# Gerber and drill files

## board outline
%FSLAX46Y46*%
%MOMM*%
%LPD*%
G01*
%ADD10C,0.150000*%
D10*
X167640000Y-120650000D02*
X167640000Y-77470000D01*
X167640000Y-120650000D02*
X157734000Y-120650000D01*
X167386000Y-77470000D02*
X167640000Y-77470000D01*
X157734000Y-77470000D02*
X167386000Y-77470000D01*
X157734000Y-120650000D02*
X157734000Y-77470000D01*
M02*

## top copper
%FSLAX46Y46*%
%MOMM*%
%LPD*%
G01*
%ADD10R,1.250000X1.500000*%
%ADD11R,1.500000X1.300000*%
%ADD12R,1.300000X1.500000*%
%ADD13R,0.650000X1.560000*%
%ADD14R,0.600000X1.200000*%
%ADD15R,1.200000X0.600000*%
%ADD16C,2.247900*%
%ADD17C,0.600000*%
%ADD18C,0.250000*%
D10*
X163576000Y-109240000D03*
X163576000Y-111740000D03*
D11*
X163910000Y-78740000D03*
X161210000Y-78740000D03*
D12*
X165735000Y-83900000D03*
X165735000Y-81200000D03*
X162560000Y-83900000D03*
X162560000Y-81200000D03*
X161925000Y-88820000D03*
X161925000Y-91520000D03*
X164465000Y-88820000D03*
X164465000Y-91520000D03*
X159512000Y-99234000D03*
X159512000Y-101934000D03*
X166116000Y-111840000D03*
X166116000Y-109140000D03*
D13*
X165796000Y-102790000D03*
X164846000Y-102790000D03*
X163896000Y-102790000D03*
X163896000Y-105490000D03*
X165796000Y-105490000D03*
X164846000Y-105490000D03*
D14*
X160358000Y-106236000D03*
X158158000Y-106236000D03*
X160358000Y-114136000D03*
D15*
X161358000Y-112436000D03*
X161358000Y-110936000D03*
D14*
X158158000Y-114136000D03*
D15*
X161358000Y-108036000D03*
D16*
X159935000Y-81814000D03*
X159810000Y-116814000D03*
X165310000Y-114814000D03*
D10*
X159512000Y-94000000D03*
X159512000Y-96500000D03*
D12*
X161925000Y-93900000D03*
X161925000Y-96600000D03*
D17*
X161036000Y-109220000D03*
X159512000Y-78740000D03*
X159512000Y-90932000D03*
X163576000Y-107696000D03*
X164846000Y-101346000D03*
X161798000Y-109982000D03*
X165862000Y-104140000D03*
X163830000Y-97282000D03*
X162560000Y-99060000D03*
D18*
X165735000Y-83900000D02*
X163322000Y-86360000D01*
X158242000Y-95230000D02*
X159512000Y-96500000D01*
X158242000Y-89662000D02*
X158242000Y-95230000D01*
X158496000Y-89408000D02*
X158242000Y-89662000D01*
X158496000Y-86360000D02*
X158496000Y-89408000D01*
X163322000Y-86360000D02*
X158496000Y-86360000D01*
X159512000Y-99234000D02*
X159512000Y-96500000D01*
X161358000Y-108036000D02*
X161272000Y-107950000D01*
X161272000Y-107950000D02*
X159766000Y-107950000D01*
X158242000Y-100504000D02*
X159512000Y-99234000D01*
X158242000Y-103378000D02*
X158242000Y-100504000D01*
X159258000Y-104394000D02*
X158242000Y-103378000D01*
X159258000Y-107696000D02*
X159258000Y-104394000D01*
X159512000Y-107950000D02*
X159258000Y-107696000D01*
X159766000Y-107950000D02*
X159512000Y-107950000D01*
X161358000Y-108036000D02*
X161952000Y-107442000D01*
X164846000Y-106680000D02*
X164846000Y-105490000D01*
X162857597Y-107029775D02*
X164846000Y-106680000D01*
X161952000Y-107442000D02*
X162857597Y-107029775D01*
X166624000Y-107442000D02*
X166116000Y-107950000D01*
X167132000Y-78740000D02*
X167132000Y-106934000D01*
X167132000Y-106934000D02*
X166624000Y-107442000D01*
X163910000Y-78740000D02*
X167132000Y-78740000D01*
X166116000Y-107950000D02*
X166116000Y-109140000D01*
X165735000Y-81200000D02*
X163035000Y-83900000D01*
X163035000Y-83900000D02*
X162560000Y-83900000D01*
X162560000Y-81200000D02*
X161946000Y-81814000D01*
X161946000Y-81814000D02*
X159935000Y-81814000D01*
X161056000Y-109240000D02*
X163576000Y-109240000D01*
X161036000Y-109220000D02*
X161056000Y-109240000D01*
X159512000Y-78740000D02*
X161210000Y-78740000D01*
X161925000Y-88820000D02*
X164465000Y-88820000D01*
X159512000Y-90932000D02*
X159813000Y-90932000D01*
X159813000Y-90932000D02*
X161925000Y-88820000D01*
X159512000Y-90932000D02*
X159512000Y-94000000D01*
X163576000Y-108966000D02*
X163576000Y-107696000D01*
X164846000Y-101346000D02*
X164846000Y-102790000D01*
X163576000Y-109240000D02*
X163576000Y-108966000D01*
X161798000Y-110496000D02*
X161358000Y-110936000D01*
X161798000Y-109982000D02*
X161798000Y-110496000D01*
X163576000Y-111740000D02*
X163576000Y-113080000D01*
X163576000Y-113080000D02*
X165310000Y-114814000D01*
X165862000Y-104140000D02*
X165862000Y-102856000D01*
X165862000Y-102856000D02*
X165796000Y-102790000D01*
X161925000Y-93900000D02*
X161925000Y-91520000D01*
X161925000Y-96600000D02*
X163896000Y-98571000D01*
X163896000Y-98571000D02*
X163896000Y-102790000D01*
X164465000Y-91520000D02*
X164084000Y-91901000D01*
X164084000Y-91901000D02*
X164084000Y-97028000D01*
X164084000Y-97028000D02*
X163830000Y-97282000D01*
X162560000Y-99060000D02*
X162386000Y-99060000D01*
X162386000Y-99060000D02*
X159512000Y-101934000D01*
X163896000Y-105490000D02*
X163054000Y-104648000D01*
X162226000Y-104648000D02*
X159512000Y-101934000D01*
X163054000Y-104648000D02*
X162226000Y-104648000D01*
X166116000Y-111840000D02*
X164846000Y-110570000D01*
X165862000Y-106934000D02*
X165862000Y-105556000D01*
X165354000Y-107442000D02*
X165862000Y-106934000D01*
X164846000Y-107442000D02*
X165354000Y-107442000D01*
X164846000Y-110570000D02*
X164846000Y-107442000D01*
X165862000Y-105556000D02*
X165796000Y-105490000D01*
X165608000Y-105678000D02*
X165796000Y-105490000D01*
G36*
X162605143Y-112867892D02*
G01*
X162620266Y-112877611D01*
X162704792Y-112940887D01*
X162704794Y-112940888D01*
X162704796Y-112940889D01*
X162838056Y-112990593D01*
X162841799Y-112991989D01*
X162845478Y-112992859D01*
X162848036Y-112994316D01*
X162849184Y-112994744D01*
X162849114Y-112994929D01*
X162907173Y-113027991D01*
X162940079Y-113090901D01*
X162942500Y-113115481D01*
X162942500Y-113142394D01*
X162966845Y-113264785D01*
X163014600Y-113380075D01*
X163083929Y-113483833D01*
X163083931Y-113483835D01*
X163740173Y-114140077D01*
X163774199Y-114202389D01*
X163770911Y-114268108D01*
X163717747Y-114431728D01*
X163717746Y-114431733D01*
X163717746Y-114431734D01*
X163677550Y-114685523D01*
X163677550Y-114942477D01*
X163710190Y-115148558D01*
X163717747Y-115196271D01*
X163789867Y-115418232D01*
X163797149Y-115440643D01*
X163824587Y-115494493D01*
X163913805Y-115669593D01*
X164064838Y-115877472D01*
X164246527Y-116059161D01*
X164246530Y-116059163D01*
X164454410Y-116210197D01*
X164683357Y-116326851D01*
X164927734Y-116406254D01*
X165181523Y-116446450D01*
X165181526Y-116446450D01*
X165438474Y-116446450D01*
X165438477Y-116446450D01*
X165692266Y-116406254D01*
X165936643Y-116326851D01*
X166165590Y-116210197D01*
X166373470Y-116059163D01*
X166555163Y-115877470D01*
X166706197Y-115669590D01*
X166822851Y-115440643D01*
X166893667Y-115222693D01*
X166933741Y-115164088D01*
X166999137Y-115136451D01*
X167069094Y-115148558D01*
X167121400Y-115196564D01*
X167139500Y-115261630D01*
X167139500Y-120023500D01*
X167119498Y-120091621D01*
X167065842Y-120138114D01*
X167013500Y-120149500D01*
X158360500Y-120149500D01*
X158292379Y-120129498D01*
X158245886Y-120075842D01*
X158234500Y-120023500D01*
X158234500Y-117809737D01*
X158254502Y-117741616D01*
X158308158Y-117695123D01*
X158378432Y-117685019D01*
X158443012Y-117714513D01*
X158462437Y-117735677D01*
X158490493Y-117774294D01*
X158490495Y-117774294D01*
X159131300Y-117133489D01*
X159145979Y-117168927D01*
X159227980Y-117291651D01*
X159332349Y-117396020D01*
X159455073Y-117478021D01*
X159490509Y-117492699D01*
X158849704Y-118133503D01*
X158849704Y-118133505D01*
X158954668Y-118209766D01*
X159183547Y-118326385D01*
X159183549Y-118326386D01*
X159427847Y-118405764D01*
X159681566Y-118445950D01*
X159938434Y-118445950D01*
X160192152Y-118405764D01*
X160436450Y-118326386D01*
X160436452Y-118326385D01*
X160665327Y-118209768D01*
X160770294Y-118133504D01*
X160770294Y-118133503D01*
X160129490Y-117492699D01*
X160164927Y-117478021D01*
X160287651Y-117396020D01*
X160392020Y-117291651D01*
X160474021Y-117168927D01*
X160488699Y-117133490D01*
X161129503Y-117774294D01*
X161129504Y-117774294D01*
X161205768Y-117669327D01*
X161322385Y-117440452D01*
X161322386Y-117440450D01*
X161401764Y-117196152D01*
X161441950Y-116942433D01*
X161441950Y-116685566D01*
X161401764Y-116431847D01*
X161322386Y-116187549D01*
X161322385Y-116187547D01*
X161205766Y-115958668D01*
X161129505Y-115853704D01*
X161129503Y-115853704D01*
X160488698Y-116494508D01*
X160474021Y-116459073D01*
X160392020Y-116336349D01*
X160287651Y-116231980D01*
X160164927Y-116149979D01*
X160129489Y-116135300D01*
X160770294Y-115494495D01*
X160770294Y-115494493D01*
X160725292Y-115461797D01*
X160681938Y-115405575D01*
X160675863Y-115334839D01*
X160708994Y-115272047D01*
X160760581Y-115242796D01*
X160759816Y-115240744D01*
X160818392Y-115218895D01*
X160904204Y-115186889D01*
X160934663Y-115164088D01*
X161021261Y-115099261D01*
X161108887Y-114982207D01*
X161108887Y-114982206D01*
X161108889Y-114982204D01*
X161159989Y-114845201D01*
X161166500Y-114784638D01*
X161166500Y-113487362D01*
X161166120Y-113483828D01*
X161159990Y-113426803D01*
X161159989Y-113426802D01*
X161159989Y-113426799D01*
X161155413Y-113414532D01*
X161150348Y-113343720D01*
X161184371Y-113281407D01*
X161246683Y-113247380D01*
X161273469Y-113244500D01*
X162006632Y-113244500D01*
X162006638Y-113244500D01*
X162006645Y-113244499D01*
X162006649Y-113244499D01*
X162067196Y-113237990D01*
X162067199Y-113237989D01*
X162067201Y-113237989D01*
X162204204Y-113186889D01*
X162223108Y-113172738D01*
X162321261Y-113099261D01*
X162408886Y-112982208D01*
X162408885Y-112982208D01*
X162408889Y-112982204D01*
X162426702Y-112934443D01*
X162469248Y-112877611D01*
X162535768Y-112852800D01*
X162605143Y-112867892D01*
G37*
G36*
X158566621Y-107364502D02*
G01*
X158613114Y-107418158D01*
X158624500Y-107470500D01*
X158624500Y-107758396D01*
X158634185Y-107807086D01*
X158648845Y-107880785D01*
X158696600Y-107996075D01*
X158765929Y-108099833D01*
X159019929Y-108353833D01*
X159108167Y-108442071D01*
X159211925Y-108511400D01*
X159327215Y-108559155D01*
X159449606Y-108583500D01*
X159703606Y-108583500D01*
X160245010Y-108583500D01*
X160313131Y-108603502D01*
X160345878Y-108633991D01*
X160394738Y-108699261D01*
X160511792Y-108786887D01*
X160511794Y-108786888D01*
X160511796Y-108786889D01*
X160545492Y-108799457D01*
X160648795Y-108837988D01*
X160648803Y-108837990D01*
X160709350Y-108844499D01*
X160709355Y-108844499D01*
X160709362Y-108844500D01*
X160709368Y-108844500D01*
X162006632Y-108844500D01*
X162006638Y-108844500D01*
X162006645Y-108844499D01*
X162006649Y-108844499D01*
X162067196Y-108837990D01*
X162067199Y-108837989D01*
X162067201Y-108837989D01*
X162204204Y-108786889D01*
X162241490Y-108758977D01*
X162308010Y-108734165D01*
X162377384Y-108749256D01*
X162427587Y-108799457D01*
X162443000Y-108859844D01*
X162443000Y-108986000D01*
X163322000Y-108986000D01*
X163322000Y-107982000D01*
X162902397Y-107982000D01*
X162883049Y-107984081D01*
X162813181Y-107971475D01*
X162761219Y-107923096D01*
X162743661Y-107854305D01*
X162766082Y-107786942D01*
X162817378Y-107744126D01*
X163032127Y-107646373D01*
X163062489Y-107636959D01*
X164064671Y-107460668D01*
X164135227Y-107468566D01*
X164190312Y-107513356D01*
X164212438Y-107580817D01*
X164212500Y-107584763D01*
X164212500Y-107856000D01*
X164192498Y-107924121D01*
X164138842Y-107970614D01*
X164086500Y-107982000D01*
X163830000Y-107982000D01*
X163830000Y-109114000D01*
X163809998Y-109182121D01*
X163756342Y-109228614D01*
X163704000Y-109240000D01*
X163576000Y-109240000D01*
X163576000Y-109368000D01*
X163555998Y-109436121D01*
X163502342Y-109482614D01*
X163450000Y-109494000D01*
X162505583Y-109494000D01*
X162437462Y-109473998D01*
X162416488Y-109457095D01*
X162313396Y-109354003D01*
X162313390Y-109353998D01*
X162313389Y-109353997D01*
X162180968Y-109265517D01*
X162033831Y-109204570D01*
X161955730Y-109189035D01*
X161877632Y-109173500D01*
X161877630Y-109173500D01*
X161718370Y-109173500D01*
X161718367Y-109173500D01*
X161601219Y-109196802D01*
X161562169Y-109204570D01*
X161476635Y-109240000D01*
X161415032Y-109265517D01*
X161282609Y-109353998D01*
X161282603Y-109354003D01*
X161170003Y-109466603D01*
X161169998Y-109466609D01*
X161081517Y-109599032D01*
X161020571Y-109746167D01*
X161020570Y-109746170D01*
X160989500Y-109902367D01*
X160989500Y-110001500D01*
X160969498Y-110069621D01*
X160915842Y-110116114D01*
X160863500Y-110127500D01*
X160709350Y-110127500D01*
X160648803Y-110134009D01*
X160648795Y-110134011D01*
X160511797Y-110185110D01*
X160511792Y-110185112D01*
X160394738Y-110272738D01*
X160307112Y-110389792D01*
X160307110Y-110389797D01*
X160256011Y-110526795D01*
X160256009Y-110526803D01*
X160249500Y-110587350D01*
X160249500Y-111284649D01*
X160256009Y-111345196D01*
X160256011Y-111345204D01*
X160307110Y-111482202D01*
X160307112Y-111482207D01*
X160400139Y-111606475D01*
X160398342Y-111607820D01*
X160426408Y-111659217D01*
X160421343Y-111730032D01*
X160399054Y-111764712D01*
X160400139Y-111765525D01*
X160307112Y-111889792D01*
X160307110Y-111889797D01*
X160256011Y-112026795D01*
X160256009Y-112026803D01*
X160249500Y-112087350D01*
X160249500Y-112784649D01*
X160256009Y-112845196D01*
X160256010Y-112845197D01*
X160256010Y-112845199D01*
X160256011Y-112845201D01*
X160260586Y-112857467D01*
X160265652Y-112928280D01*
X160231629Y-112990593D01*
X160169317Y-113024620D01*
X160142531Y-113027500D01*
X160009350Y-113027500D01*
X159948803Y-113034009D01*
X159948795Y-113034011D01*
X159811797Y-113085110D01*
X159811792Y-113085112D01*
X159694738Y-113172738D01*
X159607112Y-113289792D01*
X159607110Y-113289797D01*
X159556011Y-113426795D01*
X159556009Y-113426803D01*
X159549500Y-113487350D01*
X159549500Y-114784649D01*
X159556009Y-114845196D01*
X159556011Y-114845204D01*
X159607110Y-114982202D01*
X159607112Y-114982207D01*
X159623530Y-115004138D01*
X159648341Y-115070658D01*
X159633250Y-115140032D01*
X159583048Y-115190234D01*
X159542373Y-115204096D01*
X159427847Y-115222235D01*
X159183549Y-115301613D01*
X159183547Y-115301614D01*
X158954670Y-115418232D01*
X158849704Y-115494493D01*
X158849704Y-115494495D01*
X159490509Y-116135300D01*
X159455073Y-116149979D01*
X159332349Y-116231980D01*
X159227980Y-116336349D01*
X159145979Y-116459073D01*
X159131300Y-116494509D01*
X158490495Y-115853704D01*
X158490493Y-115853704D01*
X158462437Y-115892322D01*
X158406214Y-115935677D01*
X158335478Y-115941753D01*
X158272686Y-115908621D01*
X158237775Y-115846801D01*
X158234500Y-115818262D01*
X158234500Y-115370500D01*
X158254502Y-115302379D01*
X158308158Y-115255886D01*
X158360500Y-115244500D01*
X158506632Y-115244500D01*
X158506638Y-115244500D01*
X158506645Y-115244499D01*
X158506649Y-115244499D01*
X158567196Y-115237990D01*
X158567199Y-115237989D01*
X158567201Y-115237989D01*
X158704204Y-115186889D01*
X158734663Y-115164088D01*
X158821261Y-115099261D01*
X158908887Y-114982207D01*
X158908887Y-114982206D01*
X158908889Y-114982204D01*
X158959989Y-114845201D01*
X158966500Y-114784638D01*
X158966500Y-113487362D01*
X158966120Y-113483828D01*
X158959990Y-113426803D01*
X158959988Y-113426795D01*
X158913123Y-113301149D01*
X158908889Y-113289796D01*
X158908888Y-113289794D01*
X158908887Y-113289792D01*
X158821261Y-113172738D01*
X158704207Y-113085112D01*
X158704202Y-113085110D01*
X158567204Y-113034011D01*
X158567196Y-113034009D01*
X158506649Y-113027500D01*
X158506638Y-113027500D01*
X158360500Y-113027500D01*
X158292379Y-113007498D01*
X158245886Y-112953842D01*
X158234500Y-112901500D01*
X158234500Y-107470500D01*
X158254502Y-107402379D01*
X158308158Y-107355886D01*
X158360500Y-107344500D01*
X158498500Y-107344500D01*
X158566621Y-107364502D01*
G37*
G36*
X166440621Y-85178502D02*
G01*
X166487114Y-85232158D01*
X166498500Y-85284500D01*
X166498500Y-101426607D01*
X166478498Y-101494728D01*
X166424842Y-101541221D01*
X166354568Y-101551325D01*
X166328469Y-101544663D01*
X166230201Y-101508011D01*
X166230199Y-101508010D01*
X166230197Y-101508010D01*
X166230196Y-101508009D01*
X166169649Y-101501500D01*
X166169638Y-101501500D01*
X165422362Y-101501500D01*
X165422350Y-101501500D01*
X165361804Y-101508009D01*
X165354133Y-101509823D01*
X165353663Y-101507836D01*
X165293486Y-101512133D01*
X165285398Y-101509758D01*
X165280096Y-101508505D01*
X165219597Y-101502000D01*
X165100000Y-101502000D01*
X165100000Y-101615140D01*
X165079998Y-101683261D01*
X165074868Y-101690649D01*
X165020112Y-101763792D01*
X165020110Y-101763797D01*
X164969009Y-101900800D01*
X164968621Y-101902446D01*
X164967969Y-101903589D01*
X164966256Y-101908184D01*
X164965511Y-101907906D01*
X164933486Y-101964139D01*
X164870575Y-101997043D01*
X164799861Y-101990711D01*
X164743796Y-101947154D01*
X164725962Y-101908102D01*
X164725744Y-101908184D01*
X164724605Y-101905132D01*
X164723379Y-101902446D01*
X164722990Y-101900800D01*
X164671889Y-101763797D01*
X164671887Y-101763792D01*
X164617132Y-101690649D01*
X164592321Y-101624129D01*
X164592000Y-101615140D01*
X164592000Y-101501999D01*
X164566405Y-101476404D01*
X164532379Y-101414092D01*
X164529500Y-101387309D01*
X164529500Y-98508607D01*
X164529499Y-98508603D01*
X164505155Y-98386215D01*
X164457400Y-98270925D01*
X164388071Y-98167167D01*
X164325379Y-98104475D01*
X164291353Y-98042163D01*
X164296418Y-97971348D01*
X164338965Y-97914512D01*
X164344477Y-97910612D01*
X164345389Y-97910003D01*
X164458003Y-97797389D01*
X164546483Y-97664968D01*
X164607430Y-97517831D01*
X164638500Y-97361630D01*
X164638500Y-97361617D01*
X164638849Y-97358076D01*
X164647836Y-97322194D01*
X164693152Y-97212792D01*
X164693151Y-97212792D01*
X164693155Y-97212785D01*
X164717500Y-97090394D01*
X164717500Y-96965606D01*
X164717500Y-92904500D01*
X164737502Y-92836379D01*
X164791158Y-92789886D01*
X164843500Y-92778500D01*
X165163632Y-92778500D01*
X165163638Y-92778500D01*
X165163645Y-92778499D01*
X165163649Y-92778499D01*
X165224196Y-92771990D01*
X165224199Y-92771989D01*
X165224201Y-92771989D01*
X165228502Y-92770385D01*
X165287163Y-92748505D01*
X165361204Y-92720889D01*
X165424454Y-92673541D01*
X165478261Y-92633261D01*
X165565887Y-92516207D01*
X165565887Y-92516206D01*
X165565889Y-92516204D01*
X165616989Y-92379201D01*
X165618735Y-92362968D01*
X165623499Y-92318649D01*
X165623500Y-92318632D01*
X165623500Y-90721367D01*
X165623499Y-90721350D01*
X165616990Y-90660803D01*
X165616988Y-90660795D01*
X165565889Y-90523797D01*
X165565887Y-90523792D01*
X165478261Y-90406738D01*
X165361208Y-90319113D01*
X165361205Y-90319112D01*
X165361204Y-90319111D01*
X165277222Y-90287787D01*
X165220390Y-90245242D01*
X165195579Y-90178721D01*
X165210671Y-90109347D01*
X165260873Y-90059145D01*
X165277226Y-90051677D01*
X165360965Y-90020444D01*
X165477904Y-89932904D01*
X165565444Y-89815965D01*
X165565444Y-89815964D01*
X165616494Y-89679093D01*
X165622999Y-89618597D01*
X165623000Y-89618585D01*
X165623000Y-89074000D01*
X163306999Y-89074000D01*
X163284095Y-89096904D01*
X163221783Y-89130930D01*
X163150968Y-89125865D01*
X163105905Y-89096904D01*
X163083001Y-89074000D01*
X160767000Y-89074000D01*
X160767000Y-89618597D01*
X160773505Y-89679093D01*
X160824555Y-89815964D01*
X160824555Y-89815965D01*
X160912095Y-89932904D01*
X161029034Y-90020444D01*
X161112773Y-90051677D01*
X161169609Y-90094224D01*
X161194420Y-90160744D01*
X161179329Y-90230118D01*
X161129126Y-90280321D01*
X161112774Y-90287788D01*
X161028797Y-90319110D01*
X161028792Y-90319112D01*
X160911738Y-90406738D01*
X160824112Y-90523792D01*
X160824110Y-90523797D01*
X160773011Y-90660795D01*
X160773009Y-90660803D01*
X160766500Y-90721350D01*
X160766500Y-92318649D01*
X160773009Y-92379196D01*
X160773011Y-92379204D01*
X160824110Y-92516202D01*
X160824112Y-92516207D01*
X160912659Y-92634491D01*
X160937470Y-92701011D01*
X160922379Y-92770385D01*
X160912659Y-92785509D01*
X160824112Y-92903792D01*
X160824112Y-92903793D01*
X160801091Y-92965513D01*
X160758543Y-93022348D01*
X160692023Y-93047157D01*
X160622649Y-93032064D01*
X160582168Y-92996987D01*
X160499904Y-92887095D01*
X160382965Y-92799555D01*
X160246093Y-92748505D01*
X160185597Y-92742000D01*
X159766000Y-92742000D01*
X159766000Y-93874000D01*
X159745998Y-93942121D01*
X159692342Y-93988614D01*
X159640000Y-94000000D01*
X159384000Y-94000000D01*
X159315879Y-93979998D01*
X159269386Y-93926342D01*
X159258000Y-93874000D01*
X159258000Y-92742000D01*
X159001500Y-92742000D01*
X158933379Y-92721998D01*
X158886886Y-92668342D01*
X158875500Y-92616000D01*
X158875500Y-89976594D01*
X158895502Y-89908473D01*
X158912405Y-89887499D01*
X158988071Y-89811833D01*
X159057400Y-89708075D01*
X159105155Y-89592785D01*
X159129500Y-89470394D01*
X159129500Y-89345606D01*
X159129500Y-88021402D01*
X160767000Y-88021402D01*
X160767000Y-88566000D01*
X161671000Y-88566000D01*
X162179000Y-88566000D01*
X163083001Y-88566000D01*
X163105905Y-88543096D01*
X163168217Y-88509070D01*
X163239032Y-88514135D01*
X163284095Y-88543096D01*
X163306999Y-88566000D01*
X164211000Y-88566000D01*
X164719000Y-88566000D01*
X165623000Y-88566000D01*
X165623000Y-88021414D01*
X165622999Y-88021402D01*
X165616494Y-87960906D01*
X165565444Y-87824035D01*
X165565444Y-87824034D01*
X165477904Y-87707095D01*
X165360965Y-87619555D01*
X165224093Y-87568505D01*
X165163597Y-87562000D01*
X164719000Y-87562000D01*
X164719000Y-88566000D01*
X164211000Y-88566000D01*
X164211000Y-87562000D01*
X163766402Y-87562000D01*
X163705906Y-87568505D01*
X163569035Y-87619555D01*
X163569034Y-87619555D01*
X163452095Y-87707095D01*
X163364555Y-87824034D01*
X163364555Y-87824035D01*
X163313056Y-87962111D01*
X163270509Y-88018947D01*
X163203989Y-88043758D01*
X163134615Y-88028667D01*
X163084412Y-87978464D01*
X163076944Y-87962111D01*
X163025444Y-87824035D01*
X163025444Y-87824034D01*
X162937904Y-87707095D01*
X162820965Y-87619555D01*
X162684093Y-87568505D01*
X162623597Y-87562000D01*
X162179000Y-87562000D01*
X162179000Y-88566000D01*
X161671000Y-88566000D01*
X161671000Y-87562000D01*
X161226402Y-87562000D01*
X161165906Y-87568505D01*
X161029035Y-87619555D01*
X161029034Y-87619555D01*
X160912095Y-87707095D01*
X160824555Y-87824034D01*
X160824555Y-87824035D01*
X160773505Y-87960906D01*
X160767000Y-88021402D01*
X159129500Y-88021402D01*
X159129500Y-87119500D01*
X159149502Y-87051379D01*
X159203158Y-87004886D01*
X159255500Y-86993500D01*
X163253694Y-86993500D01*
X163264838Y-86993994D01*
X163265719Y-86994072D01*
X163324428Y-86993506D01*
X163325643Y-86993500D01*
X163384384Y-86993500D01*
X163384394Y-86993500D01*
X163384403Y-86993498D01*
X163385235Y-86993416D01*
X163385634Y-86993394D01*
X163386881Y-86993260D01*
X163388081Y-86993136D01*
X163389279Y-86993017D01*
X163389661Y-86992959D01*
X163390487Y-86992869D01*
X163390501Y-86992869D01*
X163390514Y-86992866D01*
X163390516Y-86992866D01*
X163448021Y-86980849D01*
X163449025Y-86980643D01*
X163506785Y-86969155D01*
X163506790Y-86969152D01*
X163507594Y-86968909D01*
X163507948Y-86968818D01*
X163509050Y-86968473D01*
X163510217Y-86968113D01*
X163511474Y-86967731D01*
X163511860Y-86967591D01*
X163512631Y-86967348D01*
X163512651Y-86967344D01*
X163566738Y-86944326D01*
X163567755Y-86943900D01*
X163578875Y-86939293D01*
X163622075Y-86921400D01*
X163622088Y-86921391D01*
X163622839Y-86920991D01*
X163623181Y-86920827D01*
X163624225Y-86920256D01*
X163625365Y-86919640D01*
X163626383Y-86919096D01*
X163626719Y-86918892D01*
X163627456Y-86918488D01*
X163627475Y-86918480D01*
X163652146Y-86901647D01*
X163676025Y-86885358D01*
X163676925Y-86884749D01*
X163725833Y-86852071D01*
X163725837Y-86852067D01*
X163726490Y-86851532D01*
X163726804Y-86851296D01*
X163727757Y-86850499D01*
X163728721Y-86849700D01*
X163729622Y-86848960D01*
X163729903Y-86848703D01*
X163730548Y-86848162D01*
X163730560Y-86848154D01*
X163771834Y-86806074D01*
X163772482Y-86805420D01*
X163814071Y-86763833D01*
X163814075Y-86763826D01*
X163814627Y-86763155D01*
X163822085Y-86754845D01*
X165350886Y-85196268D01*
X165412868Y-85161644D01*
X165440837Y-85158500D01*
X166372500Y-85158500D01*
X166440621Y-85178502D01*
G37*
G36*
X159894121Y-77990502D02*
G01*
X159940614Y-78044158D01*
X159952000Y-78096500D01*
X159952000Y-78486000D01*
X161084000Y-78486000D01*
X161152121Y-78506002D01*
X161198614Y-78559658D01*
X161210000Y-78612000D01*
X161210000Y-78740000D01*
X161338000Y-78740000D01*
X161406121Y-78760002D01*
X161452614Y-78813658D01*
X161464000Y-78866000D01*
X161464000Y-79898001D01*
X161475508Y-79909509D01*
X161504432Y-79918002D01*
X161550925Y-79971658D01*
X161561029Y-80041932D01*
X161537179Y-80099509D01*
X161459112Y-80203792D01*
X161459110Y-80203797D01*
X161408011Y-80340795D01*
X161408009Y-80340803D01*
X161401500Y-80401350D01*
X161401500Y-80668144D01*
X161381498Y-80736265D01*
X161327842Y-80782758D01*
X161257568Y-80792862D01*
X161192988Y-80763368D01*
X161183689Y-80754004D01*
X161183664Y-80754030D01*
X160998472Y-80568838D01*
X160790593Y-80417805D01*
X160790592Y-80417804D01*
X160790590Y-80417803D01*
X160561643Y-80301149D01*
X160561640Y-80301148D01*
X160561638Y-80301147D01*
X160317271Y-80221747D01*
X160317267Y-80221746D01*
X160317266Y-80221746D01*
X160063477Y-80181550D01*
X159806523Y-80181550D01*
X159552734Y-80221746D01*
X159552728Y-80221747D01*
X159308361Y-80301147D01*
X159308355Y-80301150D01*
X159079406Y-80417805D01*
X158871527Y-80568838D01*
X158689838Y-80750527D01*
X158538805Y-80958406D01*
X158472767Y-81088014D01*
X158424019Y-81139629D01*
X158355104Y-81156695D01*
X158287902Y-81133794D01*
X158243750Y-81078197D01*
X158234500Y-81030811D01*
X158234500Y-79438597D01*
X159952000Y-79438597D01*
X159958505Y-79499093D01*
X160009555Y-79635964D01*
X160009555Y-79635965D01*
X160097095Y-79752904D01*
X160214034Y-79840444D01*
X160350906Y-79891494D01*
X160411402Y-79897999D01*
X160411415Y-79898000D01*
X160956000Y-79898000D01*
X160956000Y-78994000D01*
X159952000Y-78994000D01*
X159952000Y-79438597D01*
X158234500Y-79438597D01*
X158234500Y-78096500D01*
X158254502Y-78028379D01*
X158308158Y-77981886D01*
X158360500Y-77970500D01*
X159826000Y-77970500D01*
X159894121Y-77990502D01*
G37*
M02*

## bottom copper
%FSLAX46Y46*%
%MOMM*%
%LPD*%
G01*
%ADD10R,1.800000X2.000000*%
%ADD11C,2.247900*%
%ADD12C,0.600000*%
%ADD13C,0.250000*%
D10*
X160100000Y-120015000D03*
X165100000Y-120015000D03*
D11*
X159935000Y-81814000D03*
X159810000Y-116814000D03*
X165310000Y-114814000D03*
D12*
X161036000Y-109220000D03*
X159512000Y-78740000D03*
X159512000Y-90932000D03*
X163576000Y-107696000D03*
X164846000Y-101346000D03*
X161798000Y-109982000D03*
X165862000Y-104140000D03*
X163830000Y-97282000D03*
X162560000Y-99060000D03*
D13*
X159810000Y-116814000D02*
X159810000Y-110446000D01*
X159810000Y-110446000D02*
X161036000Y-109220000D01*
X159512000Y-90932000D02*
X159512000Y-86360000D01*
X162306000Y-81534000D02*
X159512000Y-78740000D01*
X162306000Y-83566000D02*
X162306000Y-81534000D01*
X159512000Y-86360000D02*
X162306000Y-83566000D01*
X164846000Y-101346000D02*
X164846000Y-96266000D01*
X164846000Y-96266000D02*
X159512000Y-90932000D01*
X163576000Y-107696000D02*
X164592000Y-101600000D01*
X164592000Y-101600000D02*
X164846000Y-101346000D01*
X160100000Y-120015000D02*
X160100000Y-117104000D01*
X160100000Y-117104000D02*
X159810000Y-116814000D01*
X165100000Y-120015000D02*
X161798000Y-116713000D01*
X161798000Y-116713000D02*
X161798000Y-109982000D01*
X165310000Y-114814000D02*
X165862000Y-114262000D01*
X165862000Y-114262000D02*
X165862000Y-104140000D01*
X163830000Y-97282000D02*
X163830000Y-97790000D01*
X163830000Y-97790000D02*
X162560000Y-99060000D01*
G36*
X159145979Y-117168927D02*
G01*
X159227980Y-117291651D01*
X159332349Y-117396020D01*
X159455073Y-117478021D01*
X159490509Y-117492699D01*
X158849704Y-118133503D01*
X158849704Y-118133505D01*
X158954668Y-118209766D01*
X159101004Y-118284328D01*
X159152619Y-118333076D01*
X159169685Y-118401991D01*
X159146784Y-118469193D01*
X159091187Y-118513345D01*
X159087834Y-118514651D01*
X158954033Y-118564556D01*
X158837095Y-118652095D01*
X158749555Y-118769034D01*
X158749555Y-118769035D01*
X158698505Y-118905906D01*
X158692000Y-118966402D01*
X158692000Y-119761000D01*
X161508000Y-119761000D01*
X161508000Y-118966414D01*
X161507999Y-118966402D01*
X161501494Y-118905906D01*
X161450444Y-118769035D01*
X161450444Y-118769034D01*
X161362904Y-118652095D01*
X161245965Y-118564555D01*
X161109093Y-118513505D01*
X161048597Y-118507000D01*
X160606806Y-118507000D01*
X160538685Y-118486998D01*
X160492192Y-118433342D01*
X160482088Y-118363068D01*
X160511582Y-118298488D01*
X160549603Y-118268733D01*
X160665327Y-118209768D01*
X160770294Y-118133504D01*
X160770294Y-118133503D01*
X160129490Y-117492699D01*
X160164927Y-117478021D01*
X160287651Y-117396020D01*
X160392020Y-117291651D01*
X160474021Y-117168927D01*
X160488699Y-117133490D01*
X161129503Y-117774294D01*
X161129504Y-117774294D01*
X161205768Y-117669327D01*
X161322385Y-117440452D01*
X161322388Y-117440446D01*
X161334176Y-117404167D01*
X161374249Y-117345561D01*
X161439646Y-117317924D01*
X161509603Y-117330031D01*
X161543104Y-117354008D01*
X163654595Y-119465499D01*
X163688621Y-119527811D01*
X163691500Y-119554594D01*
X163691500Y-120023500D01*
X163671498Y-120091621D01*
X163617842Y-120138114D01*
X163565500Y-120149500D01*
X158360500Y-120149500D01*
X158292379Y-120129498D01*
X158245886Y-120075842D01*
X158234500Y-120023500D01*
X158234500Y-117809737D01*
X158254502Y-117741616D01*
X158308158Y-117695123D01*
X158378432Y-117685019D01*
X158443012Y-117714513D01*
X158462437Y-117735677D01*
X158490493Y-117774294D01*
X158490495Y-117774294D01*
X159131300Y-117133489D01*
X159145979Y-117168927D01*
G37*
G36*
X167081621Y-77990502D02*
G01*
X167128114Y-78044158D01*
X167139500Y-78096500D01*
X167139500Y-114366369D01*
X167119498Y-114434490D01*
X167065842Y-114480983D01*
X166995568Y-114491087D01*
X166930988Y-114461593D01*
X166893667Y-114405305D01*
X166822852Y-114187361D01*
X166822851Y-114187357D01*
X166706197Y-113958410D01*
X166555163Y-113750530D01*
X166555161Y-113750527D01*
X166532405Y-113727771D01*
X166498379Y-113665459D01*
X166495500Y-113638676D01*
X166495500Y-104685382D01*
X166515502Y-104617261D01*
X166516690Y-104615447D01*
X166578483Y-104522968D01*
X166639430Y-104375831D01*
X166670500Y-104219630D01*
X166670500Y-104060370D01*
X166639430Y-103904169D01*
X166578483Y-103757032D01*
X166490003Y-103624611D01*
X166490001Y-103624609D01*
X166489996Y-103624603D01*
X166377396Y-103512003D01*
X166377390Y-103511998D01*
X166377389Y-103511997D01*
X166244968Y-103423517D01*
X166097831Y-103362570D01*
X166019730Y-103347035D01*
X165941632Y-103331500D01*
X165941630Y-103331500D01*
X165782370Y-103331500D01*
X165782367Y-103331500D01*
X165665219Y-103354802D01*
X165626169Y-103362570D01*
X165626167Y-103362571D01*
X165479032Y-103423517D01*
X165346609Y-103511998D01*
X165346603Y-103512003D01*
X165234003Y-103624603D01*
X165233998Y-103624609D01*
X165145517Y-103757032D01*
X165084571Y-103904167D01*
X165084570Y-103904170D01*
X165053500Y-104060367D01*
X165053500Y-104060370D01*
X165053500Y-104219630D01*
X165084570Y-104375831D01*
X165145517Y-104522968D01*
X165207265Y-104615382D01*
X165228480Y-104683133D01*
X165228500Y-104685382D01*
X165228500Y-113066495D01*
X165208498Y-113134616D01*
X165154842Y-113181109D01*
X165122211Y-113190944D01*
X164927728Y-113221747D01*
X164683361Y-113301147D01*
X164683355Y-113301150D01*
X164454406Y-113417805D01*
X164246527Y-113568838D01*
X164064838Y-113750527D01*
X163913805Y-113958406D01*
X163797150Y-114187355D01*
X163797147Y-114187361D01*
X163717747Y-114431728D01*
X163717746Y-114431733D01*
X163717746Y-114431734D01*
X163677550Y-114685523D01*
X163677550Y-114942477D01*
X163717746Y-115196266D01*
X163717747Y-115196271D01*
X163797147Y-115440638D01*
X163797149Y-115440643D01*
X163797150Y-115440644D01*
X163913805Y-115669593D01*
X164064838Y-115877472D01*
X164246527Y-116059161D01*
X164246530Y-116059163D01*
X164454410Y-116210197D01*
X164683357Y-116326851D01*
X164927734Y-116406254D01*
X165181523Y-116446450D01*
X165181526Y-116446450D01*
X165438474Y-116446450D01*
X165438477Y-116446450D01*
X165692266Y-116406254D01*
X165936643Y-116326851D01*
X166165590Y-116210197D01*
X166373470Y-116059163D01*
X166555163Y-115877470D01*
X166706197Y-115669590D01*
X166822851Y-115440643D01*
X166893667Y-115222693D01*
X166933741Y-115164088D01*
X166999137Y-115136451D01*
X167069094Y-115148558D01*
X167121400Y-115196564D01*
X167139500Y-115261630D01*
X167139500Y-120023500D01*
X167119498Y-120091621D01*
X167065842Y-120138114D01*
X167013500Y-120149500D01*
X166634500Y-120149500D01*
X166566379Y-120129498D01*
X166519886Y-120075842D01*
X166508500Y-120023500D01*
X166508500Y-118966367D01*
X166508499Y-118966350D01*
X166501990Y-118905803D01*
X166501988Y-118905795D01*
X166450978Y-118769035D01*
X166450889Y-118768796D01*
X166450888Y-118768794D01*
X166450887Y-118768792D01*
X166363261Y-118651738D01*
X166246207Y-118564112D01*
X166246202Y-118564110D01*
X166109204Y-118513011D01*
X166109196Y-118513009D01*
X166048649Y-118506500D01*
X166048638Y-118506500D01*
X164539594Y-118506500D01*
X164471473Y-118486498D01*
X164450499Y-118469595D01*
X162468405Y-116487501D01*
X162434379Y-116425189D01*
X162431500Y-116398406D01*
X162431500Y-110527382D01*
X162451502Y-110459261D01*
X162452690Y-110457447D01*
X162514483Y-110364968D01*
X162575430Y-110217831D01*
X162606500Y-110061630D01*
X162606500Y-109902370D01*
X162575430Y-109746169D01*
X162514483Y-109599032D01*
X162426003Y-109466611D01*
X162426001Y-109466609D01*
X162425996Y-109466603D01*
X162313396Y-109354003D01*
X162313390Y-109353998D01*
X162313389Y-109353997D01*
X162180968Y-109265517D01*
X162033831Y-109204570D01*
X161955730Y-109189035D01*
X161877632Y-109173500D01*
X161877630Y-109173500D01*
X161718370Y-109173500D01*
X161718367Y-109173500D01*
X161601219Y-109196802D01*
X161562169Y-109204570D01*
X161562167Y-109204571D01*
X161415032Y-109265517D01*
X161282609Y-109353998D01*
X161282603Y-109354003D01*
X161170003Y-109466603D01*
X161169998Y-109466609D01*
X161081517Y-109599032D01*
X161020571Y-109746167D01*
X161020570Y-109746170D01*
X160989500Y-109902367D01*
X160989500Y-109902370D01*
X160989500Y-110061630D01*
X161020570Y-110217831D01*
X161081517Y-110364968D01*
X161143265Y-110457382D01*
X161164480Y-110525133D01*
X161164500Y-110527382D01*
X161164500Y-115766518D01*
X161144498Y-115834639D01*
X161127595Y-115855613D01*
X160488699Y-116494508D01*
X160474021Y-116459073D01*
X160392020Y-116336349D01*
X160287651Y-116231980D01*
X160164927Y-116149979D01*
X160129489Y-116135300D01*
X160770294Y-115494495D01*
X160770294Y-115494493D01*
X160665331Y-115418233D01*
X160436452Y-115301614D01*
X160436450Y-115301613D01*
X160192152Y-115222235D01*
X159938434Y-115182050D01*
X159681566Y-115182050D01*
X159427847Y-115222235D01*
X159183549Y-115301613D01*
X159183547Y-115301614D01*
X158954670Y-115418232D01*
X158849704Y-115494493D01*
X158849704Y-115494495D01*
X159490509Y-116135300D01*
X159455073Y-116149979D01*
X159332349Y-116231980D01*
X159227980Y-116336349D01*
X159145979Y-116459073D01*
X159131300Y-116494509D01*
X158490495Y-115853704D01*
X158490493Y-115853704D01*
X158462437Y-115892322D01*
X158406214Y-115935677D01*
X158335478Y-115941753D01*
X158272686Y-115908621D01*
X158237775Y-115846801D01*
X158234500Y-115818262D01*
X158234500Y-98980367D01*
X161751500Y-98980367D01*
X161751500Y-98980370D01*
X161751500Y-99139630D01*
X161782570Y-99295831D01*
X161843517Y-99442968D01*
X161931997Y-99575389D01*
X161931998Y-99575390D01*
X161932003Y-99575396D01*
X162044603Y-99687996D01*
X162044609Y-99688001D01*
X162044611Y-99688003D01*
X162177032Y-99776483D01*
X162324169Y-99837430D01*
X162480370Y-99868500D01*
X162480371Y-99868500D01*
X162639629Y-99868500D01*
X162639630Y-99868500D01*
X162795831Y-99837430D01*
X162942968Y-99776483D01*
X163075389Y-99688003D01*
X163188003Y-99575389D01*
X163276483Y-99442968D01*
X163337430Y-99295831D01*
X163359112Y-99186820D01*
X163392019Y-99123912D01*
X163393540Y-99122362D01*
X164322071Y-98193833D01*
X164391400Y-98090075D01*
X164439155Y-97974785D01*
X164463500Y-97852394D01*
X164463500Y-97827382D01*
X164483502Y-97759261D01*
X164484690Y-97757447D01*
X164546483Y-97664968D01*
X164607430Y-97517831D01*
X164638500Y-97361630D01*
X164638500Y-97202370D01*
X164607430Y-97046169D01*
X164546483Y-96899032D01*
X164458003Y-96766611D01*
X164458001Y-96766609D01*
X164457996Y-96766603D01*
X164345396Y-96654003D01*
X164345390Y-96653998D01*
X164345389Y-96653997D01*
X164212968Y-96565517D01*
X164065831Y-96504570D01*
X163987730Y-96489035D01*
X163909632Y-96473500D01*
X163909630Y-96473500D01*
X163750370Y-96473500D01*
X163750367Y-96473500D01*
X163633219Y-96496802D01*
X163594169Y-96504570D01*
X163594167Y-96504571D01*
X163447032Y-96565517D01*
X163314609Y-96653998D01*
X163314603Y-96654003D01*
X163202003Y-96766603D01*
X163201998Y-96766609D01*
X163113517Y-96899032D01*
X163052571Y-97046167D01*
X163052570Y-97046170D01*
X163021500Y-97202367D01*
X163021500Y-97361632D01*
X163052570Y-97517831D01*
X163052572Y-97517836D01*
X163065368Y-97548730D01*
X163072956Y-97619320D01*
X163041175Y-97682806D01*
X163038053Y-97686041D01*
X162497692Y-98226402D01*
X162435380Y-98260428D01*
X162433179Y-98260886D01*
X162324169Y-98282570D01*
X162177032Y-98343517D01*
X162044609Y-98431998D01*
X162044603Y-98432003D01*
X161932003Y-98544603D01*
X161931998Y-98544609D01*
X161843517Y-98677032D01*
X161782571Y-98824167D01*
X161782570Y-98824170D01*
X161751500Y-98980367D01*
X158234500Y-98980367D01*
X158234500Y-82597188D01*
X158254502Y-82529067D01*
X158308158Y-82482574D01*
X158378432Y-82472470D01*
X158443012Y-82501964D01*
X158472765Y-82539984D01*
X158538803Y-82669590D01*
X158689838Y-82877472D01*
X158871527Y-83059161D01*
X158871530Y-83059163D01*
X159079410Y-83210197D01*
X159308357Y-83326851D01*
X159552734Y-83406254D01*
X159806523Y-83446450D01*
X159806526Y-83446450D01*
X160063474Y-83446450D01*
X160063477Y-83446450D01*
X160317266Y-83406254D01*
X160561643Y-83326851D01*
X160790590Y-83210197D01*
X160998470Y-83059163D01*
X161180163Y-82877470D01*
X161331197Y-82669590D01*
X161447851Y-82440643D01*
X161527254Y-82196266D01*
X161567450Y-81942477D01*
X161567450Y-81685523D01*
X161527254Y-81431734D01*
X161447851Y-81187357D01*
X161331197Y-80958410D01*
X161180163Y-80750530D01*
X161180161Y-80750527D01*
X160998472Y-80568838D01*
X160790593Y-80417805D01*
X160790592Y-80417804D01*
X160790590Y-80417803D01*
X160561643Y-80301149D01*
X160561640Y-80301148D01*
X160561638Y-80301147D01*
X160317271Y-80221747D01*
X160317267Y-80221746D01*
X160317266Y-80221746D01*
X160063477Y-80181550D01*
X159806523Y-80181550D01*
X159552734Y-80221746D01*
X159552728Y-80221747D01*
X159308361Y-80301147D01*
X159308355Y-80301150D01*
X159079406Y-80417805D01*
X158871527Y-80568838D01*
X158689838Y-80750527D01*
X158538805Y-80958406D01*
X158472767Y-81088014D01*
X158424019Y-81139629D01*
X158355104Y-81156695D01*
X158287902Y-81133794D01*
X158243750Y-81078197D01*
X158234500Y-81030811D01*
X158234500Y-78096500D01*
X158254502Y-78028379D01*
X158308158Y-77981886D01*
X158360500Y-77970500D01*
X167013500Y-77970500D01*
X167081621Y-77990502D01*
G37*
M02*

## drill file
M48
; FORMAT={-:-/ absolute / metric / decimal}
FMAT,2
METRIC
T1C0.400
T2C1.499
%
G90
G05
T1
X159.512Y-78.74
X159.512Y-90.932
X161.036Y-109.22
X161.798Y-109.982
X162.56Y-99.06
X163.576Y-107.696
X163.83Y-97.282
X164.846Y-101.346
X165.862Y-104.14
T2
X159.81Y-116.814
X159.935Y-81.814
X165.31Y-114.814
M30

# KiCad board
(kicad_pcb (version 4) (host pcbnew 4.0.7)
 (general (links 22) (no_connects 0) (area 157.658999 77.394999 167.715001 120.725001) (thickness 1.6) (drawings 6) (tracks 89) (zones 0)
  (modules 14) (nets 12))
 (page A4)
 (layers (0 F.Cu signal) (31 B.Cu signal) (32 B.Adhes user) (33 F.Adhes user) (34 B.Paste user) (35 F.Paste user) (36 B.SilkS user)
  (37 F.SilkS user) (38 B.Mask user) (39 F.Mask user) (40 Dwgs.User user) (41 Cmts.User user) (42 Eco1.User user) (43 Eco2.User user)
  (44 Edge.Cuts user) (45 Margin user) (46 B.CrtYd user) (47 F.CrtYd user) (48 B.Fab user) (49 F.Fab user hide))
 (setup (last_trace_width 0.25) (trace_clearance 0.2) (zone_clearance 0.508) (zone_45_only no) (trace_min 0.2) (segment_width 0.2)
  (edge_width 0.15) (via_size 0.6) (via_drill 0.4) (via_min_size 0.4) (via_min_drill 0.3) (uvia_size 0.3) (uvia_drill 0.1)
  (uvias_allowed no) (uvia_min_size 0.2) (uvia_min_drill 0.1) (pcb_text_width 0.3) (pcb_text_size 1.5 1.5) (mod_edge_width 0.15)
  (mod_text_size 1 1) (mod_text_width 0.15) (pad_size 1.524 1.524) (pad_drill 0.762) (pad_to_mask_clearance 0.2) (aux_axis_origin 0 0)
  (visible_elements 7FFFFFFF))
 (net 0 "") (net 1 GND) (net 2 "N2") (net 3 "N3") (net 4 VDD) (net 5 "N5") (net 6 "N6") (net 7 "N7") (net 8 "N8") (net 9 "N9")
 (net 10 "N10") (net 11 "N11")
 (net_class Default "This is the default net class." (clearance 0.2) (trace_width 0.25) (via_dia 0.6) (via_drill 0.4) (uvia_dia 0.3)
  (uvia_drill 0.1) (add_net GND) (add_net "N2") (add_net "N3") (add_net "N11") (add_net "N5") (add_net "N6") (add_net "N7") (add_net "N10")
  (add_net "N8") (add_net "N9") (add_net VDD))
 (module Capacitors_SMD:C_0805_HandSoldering (layer F.Cu) (at 163.576 110.49 270)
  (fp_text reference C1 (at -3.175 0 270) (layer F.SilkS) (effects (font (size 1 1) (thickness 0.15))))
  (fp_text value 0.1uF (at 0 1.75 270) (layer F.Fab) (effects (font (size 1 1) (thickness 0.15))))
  (pad 1 smd rect (at -1.25 0 270) (size 1.5 1.25) (layers F.Cu F.Paste F.Mask) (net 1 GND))
  (pad 2 smd rect (at 1.25 0 270) (size 1.5 1.25) (layers F.Cu F.Paste F.Mask) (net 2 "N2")))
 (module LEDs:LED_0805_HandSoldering (layer F.Cu) (at 162.56 78.74 180)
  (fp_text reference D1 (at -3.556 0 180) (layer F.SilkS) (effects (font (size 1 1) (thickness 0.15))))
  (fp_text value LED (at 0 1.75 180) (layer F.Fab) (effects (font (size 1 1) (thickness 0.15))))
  (pad 1 smd rect (at -1.35 0 180) (size 1.5 1.3) (layers F.Cu F.Paste F.Mask) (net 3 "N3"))
  (pad 2 smd rect (at 1.35 0 180) (size 1.5 1.3) (layers F.Cu F.Paste F.Mask) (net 1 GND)))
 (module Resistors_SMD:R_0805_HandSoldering (layer F.Cu) (at 165.735 82.55 90)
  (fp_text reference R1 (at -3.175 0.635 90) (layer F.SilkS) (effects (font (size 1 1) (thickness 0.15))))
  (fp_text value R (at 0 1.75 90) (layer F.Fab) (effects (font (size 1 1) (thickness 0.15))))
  (pad 1 smd rect (at -1.35 0 90) (size 1.5 1.3) (layers F.Cu F.Paste F.Mask) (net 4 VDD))
  (pad 2 smd rect (at 1.35 0 90) (size 1.5 1.3) (layers F.Cu F.Paste F.Mask) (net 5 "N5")))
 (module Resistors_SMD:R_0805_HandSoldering (layer F.Cu) (at 162.56 82.55 90)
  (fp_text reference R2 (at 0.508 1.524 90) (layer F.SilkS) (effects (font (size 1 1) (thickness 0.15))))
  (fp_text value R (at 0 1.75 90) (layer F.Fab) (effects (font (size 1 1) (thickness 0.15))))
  (pad 1 smd rect (at -1.35 0 90) (size 1.5 1.3) (layers F.Cu F.Paste F.Mask) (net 5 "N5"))
  (pad 2 smd rect (at 1.35 0 90) (size 1.5 1.3) (layers F.Cu F.Paste F.Mask) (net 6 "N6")))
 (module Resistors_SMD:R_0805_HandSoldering (layer F.Cu) (at 161.925 90.17 270)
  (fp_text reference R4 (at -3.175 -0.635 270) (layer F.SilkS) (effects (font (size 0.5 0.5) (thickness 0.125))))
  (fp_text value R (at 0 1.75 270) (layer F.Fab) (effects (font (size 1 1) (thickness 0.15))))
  (pad 1 smd rect (at -1.35 0 270) (size 1.5 1.3) (layers F.Cu F.Paste F.Mask) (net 1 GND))
  (pad 2 smd rect (at 1.35 0 270) (size 1.5 1.3) (layers F.Cu F.Paste F.Mask) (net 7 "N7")))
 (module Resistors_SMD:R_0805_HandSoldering (layer F.Cu) (at 164.465 90.17 270)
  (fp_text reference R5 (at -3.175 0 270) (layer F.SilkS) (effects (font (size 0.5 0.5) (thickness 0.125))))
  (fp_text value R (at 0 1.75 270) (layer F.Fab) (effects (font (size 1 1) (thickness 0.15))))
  (pad 1 smd rect (at -1.35 0 270) (size 1.5 1.3) (layers F.Cu F.Paste F.Mask) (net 1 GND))
  (pad 2 smd rect (at 1.35 0 270) (size 1.5 1.3) (layers F.Cu F.Paste F.Mask) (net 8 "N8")))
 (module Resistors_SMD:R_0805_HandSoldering (layer F.Cu) (at 159.512 100.584 270)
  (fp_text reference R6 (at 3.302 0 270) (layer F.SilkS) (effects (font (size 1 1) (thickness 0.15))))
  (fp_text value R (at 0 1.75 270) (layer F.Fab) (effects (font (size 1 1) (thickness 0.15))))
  (pad 1 smd rect (at -1.35 0 270) (size 1.5 1.3) (layers F.Cu F.Paste F.Mask) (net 4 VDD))
  (pad 2 smd rect (at 1.35 0 270) (size 1.5 1.3) (layers F.Cu F.Paste F.Mask) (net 8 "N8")))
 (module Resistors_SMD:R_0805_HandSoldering (layer F.Cu) (at 166.116 110.49 90)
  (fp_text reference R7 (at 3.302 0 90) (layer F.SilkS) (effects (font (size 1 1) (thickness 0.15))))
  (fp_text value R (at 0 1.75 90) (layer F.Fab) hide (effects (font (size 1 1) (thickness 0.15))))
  (pad 1 smd rect (at -1.35 0 90) (size 1.5 1.3) (layers F.Cu F.Paste F.Mask) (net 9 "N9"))
  (pad 2 smd rect (at 1.35 0 90) (size 1.5 1.3) (layers F.Cu F.Paste F.Mask) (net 3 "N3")))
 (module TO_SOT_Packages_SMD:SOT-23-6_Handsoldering (layer F.Cu) (at 164.846 104.14 270)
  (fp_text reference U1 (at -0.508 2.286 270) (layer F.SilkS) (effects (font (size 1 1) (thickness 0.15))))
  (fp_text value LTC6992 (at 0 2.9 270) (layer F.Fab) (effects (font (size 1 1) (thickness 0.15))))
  (pad 1 smd rect (at -1.35 -0.95 270) (size 1.56 0.65) (layers F.Cu F.Paste F.Mask) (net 2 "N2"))
  (pad 2 smd rect (at -1.35 0 270) (size 1.56 0.65) (layers F.Cu F.Paste F.Mask) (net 1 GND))
  (pad 3 smd rect (at -1.35 0.95 270) (size 1.56 0.65) (layers F.Cu F.Paste F.Mask) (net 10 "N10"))
  (pad 4 smd rect (at 1.35 0.95 270) (size 1.56 0.65) (layers F.Cu F.Paste F.Mask) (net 8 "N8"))
  (pad 6 smd rect (at 1.35 -0.95 270) (size 1.56 0.65) (layers F.Cu F.Paste F.Mask) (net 9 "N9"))
  (pad 5 smd rect (at 1.35 0 270) (size 1.56 0.65) (layers F.Cu F.Paste F.Mask) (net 4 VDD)))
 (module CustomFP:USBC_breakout (layer B.Cu) (at 165.1 120.015 180)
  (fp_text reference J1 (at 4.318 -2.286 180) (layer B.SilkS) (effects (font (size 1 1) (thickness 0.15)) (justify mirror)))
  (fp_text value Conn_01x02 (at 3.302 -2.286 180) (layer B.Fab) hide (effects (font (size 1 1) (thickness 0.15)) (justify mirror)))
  (pad 2 smd rect (at 5 0 180) (size 1.8 2) (layers B.Cu B.Paste B.Mask) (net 1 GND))
  (pad 1 smd rect (at 0 0 180) (size 1.8 2) (layers B.Cu B.Paste B.Mask) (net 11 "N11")))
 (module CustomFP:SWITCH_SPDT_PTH (layer F.Cu) (at 159.258 110.236)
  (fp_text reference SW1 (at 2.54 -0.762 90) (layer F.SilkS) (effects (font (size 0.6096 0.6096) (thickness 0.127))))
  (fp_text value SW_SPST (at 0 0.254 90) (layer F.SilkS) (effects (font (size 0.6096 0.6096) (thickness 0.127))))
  (pad "" smd rect (at 1.1 -4 90) (size 1.2 0.6) (layers F.Cu F.Paste F.Mask) (solder_mask_margin 0.1016))
  (pad "" smd rect (at -1.1 -4 90) (size 1.2 0.6) (layers F.Cu F.Paste F.Mask) (solder_mask_margin 0.1016))
  (pad "" smd rect (at 1.1 3.9 90) (size 1.2 0.6) (layers F.Cu F.Paste F.Mask) (solder_mask_margin 0.1016))
  (pad 3 smd rect (at 2.1 2.2) (size 1.2 0.6) (layers F.Cu F.Paste F.Mask) (solder_mask_margin 0.1016))
  (pad 2 smd rect (at 2.1 0.7) (size 1.2 0.6) (layers F.Cu F.Paste F.Mask) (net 11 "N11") (solder_mask_margin 0.1016))
  (pad "" smd rect (at -1.1 3.9 90) (size 1.2 0.6) (layers F.Cu F.Paste F.Mask) (solder_mask_margin 0.1016))
  (pad 1 smd rect (at 2.1 -2.2) (size 1.2 0.6) (layers F.Cu F.Paste F.Mask) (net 4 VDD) (solder_mask_margin 0.1016)))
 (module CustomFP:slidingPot (layer F.Cu) (at 162.56 99.314 90)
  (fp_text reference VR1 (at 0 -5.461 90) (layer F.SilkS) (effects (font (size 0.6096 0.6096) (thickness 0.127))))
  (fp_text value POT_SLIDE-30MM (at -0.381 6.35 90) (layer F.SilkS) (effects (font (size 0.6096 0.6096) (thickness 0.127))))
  (pad BOTT thru_hole circle (at 17.5 -2.625 90) (size 2.2479 2.2479) (drill 1.4986) (layers *.Cu *.Mask) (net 6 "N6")
   (solder_mask_margin 0.1016))
  (pad TOP thru_hole circle (at -17.5 -2.75 90) (size 2.2479 2.2479) (drill 1.4986) (layers *.Cu *.Mask) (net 1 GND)
   (solder_mask_margin 0.1016))
  (pad WIPE thru_hole circle (at -15.5 2.75 90) (size 2.2479 2.2479) (drill 1.4986) (layers *.Cu *.Mask) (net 2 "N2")
   (solder_mask_margin 0.1016)))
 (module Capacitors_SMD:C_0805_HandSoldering (layer F.Cu) (at 159.512 95.25 270)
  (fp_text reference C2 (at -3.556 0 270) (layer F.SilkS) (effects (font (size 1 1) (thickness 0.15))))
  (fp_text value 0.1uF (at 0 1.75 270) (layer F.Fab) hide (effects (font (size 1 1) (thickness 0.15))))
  (pad 1 smd rect (at -1.25 0 270) (size 1.5 1.25) (layers F.Cu F.Paste F.Mask) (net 1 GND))
  (pad 2 smd rect (at 1.25 0 270) (size 1.5 1.25) (layers F.Cu F.Paste F.Mask) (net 4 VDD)))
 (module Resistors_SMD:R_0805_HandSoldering (layer F.Cu) (at 161.925 95.25 270)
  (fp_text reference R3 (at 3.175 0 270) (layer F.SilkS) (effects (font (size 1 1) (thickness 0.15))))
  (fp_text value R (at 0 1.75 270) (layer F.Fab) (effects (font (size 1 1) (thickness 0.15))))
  (pad 1 smd rect (at -1.35 0 270) (size 1.5 1.3) (layers F.Cu F.Paste F.Mask) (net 7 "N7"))
  (pad 2 smd rect (at 1.35 0 270) (size 1.5 1.3) (layers F.Cu F.Paste F.Mask) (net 10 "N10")))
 (gr_line (start 167.64 120.65) (end 167.64 77.47) (angle 90) (layer Edge.Cuts) (width 0.15))
 (gr_line (start 167.64 120.65) (end 157.734 120.65) (angle 90) (layer Edge.Cuts) (width 0.15))
 (gr_line (start 167.386 77.47) (end 167.64 77.47) (angle 90) (layer Edge.Cuts) (width 0.15))
 (gr_line (start 157.734 77.47) (end 167.386 77.47) (angle 90) (layer Edge.Cuts) (width 0.15))
 (gr_line (start 157.734 120.65) (end 157.734 77.47) (angle 90) (layer Edge.Cuts) (width 0.15))
 (segment (start 165.735 83.9) (end 163.322 86.36) (width 0.25) (layer F.Cu) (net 4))
 (segment (start 158.242 95.23) (end 159.512 96.5) (width 0.25) (layer F.Cu) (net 4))
 (segment (start 158.242 89.662) (end 158.242 95.23) (width 0.25) (layer F.Cu) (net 4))
 (segment (start 158.496 89.408) (end 158.242 89.662) (width 0.25) (layer F.Cu) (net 4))
 (segment (start 158.496 86.36) (end 158.496 89.408) (width 0.25) (layer F.Cu) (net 4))
 (segment (start 163.322 86.36) (end 158.496 86.36) (width 0.25) (layer F.Cu) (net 4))
 (segment (start 159.512 99.234) (end 159.512 96.5) (width 0.25) (layer F.Cu) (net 4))
 (segment (start 161.358 108.036) (end 161.272 107.95) (width 0.25) (layer F.Cu) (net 4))
 (segment (start 161.272 107.95) (end 159.766 107.95) (width 0.25) (layer F.Cu) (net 4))
 (segment (start 158.242 100.504) (end 159.512 99.234) (width 0.25) (layer F.Cu) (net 4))
 (segment (start 158.242 103.378) (end 158.242 100.504) (width 0.25) (layer F.Cu) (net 4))
 (segment (start 159.258 104.394) (end 158.242 103.378) (width 0.25) (layer F.Cu) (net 4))
 (segment (start 159.258 107.696) (end 159.258 104.394) (width 0.25) (layer F.Cu) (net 4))
 (segment (start 159.512 107.95) (end 159.258 107.696) (width 0.25) (layer F.Cu) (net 4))
 (segment (start 159.766 107.95) (end 159.512 107.95) (width 0.25) (layer F.Cu) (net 4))
 (segment (start 161.358 108.036) (end 161.952 107.442) (width 0.25) (layer F.Cu) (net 4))
 (segment (start 164.846 106.68) (end 164.846 105.49) (width 0.25) (layer F.Cu) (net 4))
 (segment (start 162.857597 107.029775) (end 164.846 106.68) (width 0.25) (layer F.Cu) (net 4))
 (segment (start 161.952 107.442) (end 162.857597 107.029775) (width 0.25) (layer F.Cu) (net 4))
 (segment (start 166.624 107.442) (end 166.116 107.95) (width 0.25) (layer F.Cu) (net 3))
 (segment (start 167.132 78.74) (end 167.132 106.934) (width 0.25) (layer F.Cu) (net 3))
 (segment (start 167.132 106.934) (end 166.624 107.442) (width 0.25) (layer F.Cu) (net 3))
 (segment (start 163.91 78.74) (end 167.132 78.74) (width 0.25) (layer F.Cu) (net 3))
 (segment (start 166.116 107.95) (end 166.116 109.14) (width 0.25) (layer F.Cu) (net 3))
 (segment (start 165.735 81.2) (end 163.035 83.9) (width 0.25) (layer F.Cu) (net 5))
 (segment (start 163.035 83.9) (end 162.56 83.9) (width 0.25) (layer F.Cu) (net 5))
 (segment (start 162.56 81.2) (end 161.946 81.814) (width 0.25) (layer F.Cu) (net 6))
 (segment (start 161.946 81.814) (end 159.935 81.814) (width 0.25) (layer F.Cu) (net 6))
 (segment (start 159.81 116.814) (end 159.81 110.446) (width 0.25) (layer B.Cu) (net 1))
 (segment (start 161.056 109.24) (end 163.576 109.24) (width 0.25) (layer F.Cu) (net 1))
 (segment (start 161.036 109.22) (end 161.056 109.24) (width 0.25) (layer F.Cu) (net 1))
 (via (at 161.036 109.22) (size 0.6) (drill 0.4) (layers F.Cu B.Cu) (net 1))
 (segment (start 159.81 110.446) (end 161.036 109.22) (width 0.25) (layer B.Cu) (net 1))
 (segment (start 159.512 90.932) (end 159.512 86.36) (width 0.25) (layer B.Cu) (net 1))
 (segment (start 159.512 78.74) (end 161.21 78.74) (width 0.25) (layer F.Cu) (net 1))
 (via (at 159.512 78.74) (size 0.6) (drill 0.4) (layers F.Cu B.Cu) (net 1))
 (segment (start 162.306 81.534) (end 159.512 78.74) (width 0.25) (layer B.Cu) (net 1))
 (segment (start 162.306 83.566) (end 162.306 81.534) (width 0.25) (layer B.Cu) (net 1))
 (segment (start 159.512 86.36) (end 162.306 83.566) (width 0.25) (layer B.Cu) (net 1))
 (segment (start 161.925 88.82) (end 164.465 88.82) (width 0.25) (layer F.Cu) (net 1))
 (segment (start 159.512 90.932) (end 159.813 90.932) (width 0.25) (layer F.Cu) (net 1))
 (segment (start 159.813 90.932) (end 161.925 88.82) (width 0.25) (layer F.Cu) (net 1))
 (segment (start 164.846 101.346) (end 164.846 96.266) (width 0.25) (layer B.Cu) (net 1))
 (segment (start 159.512 90.932) (end 159.512 94) (width 0.25) (layer F.Cu) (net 1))
 (via (at 159.512 90.932) (size 0.6) (drill 0.4) (layers F.Cu B.Cu) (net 1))
 (segment (start 164.846 96.266) (end 159.512 90.932) (width 0.25) (layer B.Cu) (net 1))
 (segment (start 163.576 107.696) (end 164.592 101.6) (width 0.25) (layer B.Cu) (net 1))
 (via (at 163.576 107.696) (size 0.6) (drill 0.4) (layers F.Cu B.Cu) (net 1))
 (segment (start 163.576 108.966) (end 163.576 107.696) (width 0.25) (layer F.Cu) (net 1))
 (segment (start 164.846 101.346) (end 164.846 102.79) (width 0.25) (layer F.Cu) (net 1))
 (via (at 164.846 101.346) (size 0.6) (drill 0.4) (layers F.Cu B.Cu) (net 1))
 (segment (start 164.592 101.6) (end 164.846 101.346) (width 0.25) (layer B.Cu) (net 1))
 (segment (start 163.576 109.24) (end 163.576 108.966) (width 0.25) (layer F.Cu) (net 1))
 (segment (start 160.1 120.015) (end 160.1 117.104) (width 0.25) (layer B.Cu) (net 1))
 (segment (start 160.1 117.104) (end 159.81 116.814) (width 0.25) (layer B.Cu) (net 1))
 (segment (start 165.1 120.015) (end 161.798 116.713) (width 0.25) (layer B.Cu) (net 11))
 (segment (start 161.798 110.496) (end 161.358 110.936) (width 0.25) (layer F.Cu) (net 11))
 (segment (start 161.798 109.982) (end 161.798 110.496) (width 0.25) (layer F.Cu) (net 11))
 (via (at 161.798 109.982) (size 0.6) (drill 0.4) (layers F.Cu B.Cu) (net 11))
 (segment (start 161.798 116.713) (end 161.798 109.982) (width 0.25) (layer B.Cu) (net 11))
 (segment (start 163.576 111.74) (end 163.576 113.08) (width 0.25) (layer F.Cu) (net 2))
 (segment (start 163.576 113.08) (end 165.31 114.814) (width 0.25) (layer F.Cu) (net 2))
 (segment (start 165.31 114.814) (end 165.862 114.262) (width 0.25) (layer B.Cu) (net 2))
 (segment (start 165.862 114.262) (end 165.862 104.14) (width 0.25) (layer B.Cu) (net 2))
 (segment (start 165.862 104.14) (end 165.862 102.856) (width 0.25) (layer F.Cu) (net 2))
 (via (at 165.862 104.14) (size 0.6) (drill 0.4) (layers F.Cu B.Cu) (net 2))
 (segment (start 165.862 102.856) (end 165.796 102.79) (width 0.25) (layer F.Cu) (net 2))
 (segment (start 161.925 93.9) (end 161.925 91.52) (width 0.25) (layer F.Cu) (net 7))
 (segment (start 161.925 96.6) (end 163.896 98.571) (width 0.25) (layer F.Cu) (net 10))
 (segment (start 163.896 98.571) (end 163.896 102.79) (width 0.25) (layer F.Cu) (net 10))
 (segment (start 164.465 91.52) (end 164.084 91.901) (width 0.25) (layer F.Cu) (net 8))
 (segment (start 164.084 91.901) (end 164.084 97.028) (width 0.25) (layer F.Cu) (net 8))
 (segment (start 164.084 97.028) (end 163.83 97.282) (width 0.25) (layer F.Cu) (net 8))
 (via (at 163.83 97.282) (size 0.6) (drill 0.4) (layers F.Cu B.Cu) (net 8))
 (segment (start 163.83 97.282) (end 163.83 97.79) (width 0.25) (layer B.Cu) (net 8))
 (segment (start 163.83 97.79) (end 162.56 99.06) (width 0.25) (layer B.Cu) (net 8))
 (via (at 162.56 99.06) (size 0.6) (drill 0.4) (layers F.Cu B.Cu) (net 8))
 (segment (start 162.56 99.06) (end 162.386 99.06) (width 0.25) (layer F.Cu) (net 8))
 (segment (start 162.386 99.06) (end 159.512 101.934) (width 0.25) (layer F.Cu) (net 8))
 (segment (start 163.896 105.49) (end 163.054 104.648) (width 0.25) (layer F.Cu) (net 8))
 (segment (start 162.226 104.648) (end 159.512 101.934) (width 0.25) (layer F.Cu) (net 8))
 (segment (start 163.054 104.648) (end 162.226 104.648) (width 0.25) (layer F.Cu) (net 8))
 (segment (start 166.116 111.84) (end 164.846 110.57) (width 0.25) (layer F.Cu) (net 9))
 (segment (start 165.862 106.934) (end 165.862 105.556) (width 0.25) (layer F.Cu) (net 9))
 (segment (start 165.354 107.442) (end 165.862 106.934) (width 0.25) (layer F.Cu) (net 9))
 (segment (start 164.846 107.442) (end 165.354 107.442) (width 0.25) (layer F.Cu) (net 9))
 (segment (start 164.846 110.57) (end 164.846 107.442) (width 0.25) (layer F.Cu) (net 9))
 (segment (start 165.862 105.556) (end 165.796 105.49) (width 0.25) (layer F.Cu) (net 9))
 (segment (start 165.608 105.678) (end 165.796 105.49) (width 0.25) (layer F.Cu) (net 9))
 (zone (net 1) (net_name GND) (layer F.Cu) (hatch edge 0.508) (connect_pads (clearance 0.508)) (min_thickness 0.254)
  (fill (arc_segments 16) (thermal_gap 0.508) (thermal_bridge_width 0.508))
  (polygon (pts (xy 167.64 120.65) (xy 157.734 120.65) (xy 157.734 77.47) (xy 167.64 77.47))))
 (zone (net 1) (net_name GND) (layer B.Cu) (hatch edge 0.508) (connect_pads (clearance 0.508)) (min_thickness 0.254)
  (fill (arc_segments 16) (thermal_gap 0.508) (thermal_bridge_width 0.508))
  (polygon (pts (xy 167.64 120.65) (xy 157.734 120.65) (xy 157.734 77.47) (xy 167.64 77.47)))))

